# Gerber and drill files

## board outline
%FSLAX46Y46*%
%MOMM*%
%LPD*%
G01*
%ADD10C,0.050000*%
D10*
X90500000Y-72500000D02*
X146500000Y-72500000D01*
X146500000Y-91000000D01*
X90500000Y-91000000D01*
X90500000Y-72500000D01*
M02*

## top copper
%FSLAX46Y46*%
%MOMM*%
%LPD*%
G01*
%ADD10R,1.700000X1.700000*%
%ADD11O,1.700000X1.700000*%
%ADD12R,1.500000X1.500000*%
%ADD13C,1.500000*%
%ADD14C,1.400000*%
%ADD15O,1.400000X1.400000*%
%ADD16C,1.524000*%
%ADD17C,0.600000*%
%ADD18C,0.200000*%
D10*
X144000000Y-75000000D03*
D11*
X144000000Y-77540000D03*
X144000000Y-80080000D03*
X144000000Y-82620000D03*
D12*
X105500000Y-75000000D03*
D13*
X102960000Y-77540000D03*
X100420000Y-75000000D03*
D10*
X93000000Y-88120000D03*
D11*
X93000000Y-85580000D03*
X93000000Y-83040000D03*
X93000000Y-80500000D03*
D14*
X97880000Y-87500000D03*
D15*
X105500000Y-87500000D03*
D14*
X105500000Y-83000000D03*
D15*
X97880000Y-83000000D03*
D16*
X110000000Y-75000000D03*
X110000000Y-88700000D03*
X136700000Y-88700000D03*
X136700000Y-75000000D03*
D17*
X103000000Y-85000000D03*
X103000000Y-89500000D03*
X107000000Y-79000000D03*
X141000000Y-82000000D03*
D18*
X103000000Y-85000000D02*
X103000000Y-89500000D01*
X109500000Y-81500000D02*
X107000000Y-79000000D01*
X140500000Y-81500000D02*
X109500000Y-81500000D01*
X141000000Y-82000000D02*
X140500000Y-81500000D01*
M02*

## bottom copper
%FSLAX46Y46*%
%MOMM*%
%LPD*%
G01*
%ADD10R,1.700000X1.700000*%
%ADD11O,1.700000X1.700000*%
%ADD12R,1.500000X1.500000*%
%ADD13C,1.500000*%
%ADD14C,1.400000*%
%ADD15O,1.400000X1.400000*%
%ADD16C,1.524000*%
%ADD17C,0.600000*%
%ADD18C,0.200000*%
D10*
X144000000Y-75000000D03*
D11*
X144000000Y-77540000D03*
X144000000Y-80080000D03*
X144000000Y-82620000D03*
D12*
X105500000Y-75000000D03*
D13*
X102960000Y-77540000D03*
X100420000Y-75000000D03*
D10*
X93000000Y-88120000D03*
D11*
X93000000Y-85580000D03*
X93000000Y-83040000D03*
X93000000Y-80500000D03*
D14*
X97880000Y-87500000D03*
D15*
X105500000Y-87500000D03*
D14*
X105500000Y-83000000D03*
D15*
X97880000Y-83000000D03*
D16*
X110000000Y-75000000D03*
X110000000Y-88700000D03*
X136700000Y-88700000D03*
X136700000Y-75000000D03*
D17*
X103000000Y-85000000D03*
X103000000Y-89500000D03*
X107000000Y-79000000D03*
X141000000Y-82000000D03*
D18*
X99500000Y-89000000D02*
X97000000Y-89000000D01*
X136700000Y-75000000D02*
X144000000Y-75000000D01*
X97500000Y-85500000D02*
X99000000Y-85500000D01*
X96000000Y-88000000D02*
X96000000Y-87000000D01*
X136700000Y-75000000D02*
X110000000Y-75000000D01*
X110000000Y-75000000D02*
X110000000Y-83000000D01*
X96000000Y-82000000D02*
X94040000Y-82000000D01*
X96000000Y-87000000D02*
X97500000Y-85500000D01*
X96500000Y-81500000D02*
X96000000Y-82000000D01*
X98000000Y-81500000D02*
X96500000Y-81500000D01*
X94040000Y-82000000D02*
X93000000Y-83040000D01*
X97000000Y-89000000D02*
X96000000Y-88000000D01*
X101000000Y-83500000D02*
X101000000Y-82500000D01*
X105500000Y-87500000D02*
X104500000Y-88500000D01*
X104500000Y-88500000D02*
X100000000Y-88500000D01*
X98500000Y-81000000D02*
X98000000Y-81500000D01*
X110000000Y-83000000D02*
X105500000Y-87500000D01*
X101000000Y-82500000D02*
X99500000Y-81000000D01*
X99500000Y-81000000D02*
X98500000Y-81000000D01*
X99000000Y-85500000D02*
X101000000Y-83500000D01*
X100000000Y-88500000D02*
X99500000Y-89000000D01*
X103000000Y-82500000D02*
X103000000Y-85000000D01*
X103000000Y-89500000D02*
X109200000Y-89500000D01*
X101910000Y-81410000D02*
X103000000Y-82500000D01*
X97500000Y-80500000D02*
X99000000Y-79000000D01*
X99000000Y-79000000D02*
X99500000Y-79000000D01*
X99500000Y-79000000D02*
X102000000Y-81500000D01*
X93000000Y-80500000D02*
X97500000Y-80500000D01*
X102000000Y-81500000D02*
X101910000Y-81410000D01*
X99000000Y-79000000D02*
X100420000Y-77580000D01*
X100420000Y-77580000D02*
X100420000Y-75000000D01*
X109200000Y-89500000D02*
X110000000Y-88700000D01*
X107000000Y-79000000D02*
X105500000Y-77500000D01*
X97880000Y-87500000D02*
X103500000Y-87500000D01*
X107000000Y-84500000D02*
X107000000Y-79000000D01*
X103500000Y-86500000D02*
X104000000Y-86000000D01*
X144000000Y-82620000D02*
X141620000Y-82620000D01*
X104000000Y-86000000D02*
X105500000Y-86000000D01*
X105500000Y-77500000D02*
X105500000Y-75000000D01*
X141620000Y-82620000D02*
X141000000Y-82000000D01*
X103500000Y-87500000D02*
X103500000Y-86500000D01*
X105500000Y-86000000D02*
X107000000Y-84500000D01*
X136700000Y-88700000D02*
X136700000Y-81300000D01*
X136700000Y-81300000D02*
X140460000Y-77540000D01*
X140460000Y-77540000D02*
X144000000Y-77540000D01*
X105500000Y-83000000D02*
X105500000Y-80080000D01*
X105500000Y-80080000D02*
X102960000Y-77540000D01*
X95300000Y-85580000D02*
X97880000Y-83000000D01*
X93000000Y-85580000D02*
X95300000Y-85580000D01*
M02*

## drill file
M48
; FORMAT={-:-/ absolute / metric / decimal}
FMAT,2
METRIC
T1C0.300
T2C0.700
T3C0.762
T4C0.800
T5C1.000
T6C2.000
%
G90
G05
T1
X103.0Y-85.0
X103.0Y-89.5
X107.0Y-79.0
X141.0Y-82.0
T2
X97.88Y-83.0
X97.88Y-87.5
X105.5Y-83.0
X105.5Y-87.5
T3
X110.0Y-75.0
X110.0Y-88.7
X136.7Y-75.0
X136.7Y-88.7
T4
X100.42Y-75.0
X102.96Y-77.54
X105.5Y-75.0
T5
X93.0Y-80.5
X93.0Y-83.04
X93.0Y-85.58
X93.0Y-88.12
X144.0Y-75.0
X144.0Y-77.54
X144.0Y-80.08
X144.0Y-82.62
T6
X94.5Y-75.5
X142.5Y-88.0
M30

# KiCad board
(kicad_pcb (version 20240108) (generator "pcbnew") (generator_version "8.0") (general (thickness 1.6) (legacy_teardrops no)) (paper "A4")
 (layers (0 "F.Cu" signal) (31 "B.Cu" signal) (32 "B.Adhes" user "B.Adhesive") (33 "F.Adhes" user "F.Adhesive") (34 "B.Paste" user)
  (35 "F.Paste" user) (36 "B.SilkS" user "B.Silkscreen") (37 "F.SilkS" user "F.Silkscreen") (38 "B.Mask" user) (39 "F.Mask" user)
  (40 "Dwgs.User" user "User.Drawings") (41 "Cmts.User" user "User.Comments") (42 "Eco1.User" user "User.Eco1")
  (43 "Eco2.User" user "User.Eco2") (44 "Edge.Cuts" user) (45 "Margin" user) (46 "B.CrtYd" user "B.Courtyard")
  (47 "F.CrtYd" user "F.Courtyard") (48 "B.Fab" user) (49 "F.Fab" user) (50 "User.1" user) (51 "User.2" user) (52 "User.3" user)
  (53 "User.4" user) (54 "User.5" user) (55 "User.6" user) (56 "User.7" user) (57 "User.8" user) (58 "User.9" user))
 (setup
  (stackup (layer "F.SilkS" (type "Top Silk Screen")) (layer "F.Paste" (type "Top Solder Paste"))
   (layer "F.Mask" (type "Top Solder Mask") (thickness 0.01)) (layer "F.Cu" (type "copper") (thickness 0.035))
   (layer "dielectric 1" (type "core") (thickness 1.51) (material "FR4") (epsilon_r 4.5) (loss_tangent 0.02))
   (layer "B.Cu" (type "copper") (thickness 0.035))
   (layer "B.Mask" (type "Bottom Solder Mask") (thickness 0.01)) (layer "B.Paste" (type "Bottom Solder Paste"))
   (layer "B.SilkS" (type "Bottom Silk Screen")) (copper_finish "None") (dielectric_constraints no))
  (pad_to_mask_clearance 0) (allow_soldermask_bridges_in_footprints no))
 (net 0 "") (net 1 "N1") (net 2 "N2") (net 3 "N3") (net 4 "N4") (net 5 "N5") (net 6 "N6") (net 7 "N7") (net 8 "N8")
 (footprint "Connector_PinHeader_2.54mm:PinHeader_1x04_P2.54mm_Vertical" (layer "F.Cu") (at 144 75)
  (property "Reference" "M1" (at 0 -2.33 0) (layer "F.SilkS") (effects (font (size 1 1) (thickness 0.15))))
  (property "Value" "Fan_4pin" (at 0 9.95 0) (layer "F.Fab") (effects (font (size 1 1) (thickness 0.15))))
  (pad "1" thru_hole rect (at 0 0) (size 1.7 1.7) (drill 1) (layers "*.Cu" "*.Mask") (remove_unused_layers no) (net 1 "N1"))
  (pad "2" thru_hole oval (at 0 2.54) (size 1.7 1.7) (drill 1) (layers "*.Cu" "*.Mask") (remove_unused_layers no) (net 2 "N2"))
  (pad "3" thru_hole oval (at 0 5.08) (size 1.7 1.7) (drill 1) (layers "*.Cu" "*.Mask") (remove_unused_layers no) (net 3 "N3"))
  (pad "4" thru_hole oval (at 0 7.62) (size 1.7 1.7) (drill 1) (layers "*.Cu" "*.Mask") (remove_unused_layers no) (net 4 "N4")))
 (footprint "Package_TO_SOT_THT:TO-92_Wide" (layer "F.Cu") (at 105.5 75 180)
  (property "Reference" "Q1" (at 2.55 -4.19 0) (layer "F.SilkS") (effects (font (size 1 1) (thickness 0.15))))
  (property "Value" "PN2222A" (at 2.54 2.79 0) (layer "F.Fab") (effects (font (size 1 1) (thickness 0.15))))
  (pad "1" thru_hole rect (at 0 0 180) (size 1.5 1.5) (drill 0.8) (layers "*.Cu" "*.Mask") (remove_unused_layers no) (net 4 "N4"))
  (pad "2" thru_hole circle (at 2.54 -2.54 180) (size 1.5 1.5) (drill 0.8) (layers "*.Cu" "*.Mask") (remove_unused_layers no) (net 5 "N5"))
  (pad "3" thru_hole circle (at 5.08 0 180) (size 1.5 1.5) (drill 0.8) (layers "*.Cu" "*.Mask") (remove_unused_layers no) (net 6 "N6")))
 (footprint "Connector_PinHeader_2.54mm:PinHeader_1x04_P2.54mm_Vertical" (layer "F.Cu") (at 93 88.12 180)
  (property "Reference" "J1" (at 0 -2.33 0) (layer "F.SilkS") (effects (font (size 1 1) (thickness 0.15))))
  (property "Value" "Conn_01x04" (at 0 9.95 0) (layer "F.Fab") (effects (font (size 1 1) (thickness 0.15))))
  (pad "1" thru_hole rect (at 0 0 180) (size 1.7 1.7) (drill 1) (layers "*.Cu" "*.Mask") (remove_unused_layers no) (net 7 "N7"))
  (pad "2" thru_hole oval (at 0 2.54 180) (size 1.7 1.7) (drill 1) (layers "*.Cu" "*.Mask") (remove_unused_layers no) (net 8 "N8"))
  (pad "3" thru_hole oval (at 0 5.08 180) (size 1.7 1.7) (drill 1) (layers "*.Cu" "*.Mask") (remove_unused_layers no) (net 1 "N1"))
  (pad "4" thru_hole oval (at 0 7.62 180) (size 1.7 1.7) (drill 1) (layers "*.Cu" "*.Mask") (remove_unused_layers no) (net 6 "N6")))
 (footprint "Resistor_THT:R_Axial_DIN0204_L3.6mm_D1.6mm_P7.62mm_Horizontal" (layer "F.Cu") (at 97.88 87.5)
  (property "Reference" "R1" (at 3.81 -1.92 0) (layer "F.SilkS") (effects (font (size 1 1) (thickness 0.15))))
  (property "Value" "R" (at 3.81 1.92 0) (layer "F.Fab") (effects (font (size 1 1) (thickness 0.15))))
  (pad "1" thru_hole circle (at 0 0) (size 1.4 1.4) (drill 0.7) (layers "*.Cu" "*.Mask") (remove_unused_layers no) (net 4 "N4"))
  (pad "2" thru_hole oval (at 7.62 0) (size 1.4 1.4) (drill 0.7) (layers "*.Cu" "*.Mask") (remove_unused_layers no) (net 1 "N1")))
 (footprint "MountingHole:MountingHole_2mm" (layer "F.Cu") (at 94.5 75.5)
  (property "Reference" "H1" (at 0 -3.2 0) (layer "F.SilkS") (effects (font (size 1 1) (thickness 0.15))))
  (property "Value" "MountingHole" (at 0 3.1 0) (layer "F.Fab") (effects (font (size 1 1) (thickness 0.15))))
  (pad "" np_thru_hole circle (at 0 0) (size 2 2) (drill 2) (layers "*.Cu" "*.Mask")))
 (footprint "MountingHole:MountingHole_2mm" (layer "F.Cu") (at 142.5 88)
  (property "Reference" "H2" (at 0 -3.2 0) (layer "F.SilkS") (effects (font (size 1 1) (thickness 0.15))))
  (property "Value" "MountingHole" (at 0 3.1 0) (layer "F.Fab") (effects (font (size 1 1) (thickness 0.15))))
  (pad "" np_thru_hole circle (at 0 0) (size 2 2) (drill 2) (layers "*.Cu" "*.Mask")))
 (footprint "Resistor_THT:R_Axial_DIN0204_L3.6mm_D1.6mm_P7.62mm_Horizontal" (layer "F.Cu") (at 105.5 83 180)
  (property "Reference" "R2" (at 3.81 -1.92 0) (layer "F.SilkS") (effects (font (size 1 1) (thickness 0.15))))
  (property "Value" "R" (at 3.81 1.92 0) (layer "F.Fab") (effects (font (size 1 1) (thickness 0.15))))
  (pad "1" thru_hole circle (at 0 0 180) (size 1.4 1.4) (drill 0.7) (layers "*.Cu" "*.Mask") (remove_unused_layers no) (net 5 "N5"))
  (pad "2" thru_hole oval (at 7.62 0 180) (size 1.4 1.4) (drill 0.7) (layers "*.Cu" "*.Mask") (remove_unused_layers no) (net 8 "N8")))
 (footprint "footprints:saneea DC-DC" (layer "F.Cu") (at 110 75)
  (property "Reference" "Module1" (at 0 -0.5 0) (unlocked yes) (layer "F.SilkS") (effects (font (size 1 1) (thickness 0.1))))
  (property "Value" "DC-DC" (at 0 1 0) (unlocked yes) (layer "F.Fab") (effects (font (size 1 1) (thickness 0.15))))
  (pad "1" thru_hole circle (at 0 0) (size 1.524 1.524) (drill 0.762) (layers "*.Cu" "*.Mask") (remove_unused_layers no) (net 1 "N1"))
  (pad "2" thru_hole circle (at 0 13.7) (size 1.524 1.524) (drill 0.762) (layers "*.Cu" "*.Mask") (remove_unused_layers no) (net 6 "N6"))
  (pad "3" thru_hole circle (at 26.7 13.7) (size 1.524 1.524) (drill 0.762) (layers "*.Cu" "*.Mask") (remove_unused_layers no) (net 2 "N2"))
  (pad "4" thru_hole circle (at 26.7 0 90) (size 1.524 1.524) (drill 0.762) (layers "*.Cu" "*.Mask") (remove_unused_layers no) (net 1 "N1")))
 (gr_rect (start 90.5 72.5) (end 146.5 91) (stroke (width 0.05) (type default)) (fill none) (layer "Edge.Cuts"))
 (segment (start 99.5 89) (end 97 89) (width 0.2) (layer "B.Cu") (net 1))
 (segment (start 136.7 75) (end 144 75) (width 0.2) (layer "B.Cu") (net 1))
 (segment (start 97.5 85.5) (end 99 85.5) (width 0.2) (layer "B.Cu") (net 1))
 (segment (start 96 88) (end 96 87) (width 0.2) (layer "B.Cu") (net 1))
 (segment (start 136.7 75) (end 110 75) (width 0.2) (layer "B.Cu") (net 1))
 (segment (start 110 75) (end 110 83) (width 0.2) (layer "B.Cu") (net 1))
 (segment (start 96 82) (end 94.04 82) (width 0.2) (layer "B.Cu") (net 1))
 (segment (start 96 87) (end 97.5 85.5) (width 0.2) (layer "B.Cu") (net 1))
 (segment (start 96.5 81.5) (end 96 82) (width 0.2) (layer "B.Cu") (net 1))
 (segment (start 98 81.5) (end 96.5 81.5) (width 0.2) (layer "B.Cu") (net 1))
 (segment (start 94.04 82) (end 93 83.04) (width 0.2) (layer "B.Cu") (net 1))
 (segment (start 97 89) (end 96 88) (width 0.2) (layer "B.Cu") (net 1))
 (segment (start 101 83.5) (end 101 82.5) (width 0.2) (layer "B.Cu") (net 1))
 (segment (start 105.5 87.5) (end 104.5 88.5) (width 0.2) (layer "B.Cu") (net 1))
 (segment (start 104.5 88.5) (end 100 88.5) (width 0.2) (layer "B.Cu") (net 1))
 (segment (start 98.5 81) (end 98 81.5) (width 0.2) (layer "B.Cu") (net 1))
 (segment (start 110 83) (end 105.5 87.5) (width 0.2) (layer "B.Cu") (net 1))
 (segment (start 101 82.5) (end 99.5 81) (width 0.2) (layer "B.Cu") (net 1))
 (segment (start 99.5 81) (end 98.5 81) (width 0.2) (layer "B.Cu") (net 1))
 (segment (start 99 85.5) (end 101 83.5) (width 0.2) (layer "B.Cu") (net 1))
 (segment (start 100 88.5) (end 99.5 89) (width 0.2) (layer "B.Cu") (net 1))
 (segment (start 103 85) (end 103 89.5) (width 0.2) (layer "F.Cu") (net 6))
 (via (at 103 85) (size 0.6) (drill 0.3) (layers "F.Cu" "B.Cu") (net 6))
 (via (at 103 89.5) (size 0.6) (drill 0.3) (layers "F.Cu" "B.Cu") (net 6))
 (segment (start 103 82.5) (end 103 85) (width 0.2) (layer "B.Cu") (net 6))
 (segment (start 103 89.5) (end 109.2 89.5) (width 0.2) (layer "B.Cu") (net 6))
 (segment (start 101.91 81.41) (end 103 82.5) (width 0.2) (layer "B.Cu") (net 6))
 (segment (start 97.5 80.5) (end 99 79) (width 0.2) (layer "B.Cu") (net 6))
 (segment (start 99 79) (end 99.5 79) (width 0.2) (layer "B.Cu") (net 6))
 (segment (start 99.5 79) (end 102 81.5) (width 0.2) (layer "B.Cu") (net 6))
 (segment (start 93 80.5) (end 97.5 80.5) (width 0.2) (layer "B.Cu") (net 6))
 (segment (start 102 81.5) (end 101.91 81.41) (width 0.2) (layer "B.Cu") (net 6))
 (segment (start 99 79) (end 100.42 77.58) (width 0.2) (layer "B.Cu") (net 6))
 (segment (start 100.42 77.58) (end 100.42 75) (width 0.2) (layer "B.Cu") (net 6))
 (segment (start 109.2 89.5) (end 110 88.7) (width 0.2) (layer "B.Cu") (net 6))
 (segment (start 109.5 81.5) (end 107 79) (width 0.2) (layer "F.Cu") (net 4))
 (segment (start 140.5 81.5) (end 109.5 81.5) (width 0.2) (layer "F.Cu") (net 4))
 (segment (start 141 82) (end 140.5 81.5) (width 0.2) (layer "F.Cu") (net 4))
 (via (at 107 79) (size 0.6) (drill 0.3) (layers "F.Cu" "B.Cu") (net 4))
 (via (at 141 82) (size 0.6) (drill 0.3) (layers "F.Cu" "B.Cu") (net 4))
 (segment (start 107 79) (end 105.5 77.5) (width 0.2) (layer "B.Cu") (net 4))
 (segment (start 97.88 87.5) (end 103.5 87.5) (width 0.2) (layer "B.Cu") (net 4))
 (segment (start 107 84.5) (end 107 79) (width 0.2) (layer "B.Cu") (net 4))
 (segment (start 103.5 86.5) (end 104 86) (width 0.2) (layer "B.Cu") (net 4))
 (segment (start 144 82.62) (end 141.62 82.62) (width 0.2) (layer "B.Cu") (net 4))
 (segment (start 104 86) (end 105.5 86) (width 0.2) (layer "B.Cu") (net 4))
 (segment (start 105.5 77.5) (end 105.5 75) (width 0.2) (layer "B.Cu") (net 4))
 (segment (start 141.62 82.62) (end 141 82) (width 0.2) (layer "B.Cu") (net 4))
 (segment (start 103.5 87.5) (end 103.5 86.5) (width 0.2) (layer "B.Cu") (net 4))
 (segment (start 105.5 86) (end 107 84.5) (width 0.2) (layer "B.Cu") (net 4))
 (segment (start 136.7 88.7) (end 136.7 81.3) (width 0.2) (layer "B.Cu") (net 2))
 (segment (start 136.7 81.3) (end 140.46 77.54) (width 0.2) (layer "B.Cu") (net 2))
 (segment (start 140.46 77.54) (end 144 77.54) (width 0.2) (layer "B.Cu") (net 2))
 (segment (start 105.5 83) (end 105.5 80.08) (width 0.2) (layer "B.Cu") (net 5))
 (segment (start 105.5 80.08) (end 102.96 77.54) (width 0.2) (layer "B.Cu") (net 5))
 (segment (start 95.3 85.58) (end 97.88 83) (width 0.2) (layer "B.Cu") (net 8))
 (segment (start 93 85.58) (end 95.3 85.58) (width 0.2) (layer "B.Cu") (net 8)))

